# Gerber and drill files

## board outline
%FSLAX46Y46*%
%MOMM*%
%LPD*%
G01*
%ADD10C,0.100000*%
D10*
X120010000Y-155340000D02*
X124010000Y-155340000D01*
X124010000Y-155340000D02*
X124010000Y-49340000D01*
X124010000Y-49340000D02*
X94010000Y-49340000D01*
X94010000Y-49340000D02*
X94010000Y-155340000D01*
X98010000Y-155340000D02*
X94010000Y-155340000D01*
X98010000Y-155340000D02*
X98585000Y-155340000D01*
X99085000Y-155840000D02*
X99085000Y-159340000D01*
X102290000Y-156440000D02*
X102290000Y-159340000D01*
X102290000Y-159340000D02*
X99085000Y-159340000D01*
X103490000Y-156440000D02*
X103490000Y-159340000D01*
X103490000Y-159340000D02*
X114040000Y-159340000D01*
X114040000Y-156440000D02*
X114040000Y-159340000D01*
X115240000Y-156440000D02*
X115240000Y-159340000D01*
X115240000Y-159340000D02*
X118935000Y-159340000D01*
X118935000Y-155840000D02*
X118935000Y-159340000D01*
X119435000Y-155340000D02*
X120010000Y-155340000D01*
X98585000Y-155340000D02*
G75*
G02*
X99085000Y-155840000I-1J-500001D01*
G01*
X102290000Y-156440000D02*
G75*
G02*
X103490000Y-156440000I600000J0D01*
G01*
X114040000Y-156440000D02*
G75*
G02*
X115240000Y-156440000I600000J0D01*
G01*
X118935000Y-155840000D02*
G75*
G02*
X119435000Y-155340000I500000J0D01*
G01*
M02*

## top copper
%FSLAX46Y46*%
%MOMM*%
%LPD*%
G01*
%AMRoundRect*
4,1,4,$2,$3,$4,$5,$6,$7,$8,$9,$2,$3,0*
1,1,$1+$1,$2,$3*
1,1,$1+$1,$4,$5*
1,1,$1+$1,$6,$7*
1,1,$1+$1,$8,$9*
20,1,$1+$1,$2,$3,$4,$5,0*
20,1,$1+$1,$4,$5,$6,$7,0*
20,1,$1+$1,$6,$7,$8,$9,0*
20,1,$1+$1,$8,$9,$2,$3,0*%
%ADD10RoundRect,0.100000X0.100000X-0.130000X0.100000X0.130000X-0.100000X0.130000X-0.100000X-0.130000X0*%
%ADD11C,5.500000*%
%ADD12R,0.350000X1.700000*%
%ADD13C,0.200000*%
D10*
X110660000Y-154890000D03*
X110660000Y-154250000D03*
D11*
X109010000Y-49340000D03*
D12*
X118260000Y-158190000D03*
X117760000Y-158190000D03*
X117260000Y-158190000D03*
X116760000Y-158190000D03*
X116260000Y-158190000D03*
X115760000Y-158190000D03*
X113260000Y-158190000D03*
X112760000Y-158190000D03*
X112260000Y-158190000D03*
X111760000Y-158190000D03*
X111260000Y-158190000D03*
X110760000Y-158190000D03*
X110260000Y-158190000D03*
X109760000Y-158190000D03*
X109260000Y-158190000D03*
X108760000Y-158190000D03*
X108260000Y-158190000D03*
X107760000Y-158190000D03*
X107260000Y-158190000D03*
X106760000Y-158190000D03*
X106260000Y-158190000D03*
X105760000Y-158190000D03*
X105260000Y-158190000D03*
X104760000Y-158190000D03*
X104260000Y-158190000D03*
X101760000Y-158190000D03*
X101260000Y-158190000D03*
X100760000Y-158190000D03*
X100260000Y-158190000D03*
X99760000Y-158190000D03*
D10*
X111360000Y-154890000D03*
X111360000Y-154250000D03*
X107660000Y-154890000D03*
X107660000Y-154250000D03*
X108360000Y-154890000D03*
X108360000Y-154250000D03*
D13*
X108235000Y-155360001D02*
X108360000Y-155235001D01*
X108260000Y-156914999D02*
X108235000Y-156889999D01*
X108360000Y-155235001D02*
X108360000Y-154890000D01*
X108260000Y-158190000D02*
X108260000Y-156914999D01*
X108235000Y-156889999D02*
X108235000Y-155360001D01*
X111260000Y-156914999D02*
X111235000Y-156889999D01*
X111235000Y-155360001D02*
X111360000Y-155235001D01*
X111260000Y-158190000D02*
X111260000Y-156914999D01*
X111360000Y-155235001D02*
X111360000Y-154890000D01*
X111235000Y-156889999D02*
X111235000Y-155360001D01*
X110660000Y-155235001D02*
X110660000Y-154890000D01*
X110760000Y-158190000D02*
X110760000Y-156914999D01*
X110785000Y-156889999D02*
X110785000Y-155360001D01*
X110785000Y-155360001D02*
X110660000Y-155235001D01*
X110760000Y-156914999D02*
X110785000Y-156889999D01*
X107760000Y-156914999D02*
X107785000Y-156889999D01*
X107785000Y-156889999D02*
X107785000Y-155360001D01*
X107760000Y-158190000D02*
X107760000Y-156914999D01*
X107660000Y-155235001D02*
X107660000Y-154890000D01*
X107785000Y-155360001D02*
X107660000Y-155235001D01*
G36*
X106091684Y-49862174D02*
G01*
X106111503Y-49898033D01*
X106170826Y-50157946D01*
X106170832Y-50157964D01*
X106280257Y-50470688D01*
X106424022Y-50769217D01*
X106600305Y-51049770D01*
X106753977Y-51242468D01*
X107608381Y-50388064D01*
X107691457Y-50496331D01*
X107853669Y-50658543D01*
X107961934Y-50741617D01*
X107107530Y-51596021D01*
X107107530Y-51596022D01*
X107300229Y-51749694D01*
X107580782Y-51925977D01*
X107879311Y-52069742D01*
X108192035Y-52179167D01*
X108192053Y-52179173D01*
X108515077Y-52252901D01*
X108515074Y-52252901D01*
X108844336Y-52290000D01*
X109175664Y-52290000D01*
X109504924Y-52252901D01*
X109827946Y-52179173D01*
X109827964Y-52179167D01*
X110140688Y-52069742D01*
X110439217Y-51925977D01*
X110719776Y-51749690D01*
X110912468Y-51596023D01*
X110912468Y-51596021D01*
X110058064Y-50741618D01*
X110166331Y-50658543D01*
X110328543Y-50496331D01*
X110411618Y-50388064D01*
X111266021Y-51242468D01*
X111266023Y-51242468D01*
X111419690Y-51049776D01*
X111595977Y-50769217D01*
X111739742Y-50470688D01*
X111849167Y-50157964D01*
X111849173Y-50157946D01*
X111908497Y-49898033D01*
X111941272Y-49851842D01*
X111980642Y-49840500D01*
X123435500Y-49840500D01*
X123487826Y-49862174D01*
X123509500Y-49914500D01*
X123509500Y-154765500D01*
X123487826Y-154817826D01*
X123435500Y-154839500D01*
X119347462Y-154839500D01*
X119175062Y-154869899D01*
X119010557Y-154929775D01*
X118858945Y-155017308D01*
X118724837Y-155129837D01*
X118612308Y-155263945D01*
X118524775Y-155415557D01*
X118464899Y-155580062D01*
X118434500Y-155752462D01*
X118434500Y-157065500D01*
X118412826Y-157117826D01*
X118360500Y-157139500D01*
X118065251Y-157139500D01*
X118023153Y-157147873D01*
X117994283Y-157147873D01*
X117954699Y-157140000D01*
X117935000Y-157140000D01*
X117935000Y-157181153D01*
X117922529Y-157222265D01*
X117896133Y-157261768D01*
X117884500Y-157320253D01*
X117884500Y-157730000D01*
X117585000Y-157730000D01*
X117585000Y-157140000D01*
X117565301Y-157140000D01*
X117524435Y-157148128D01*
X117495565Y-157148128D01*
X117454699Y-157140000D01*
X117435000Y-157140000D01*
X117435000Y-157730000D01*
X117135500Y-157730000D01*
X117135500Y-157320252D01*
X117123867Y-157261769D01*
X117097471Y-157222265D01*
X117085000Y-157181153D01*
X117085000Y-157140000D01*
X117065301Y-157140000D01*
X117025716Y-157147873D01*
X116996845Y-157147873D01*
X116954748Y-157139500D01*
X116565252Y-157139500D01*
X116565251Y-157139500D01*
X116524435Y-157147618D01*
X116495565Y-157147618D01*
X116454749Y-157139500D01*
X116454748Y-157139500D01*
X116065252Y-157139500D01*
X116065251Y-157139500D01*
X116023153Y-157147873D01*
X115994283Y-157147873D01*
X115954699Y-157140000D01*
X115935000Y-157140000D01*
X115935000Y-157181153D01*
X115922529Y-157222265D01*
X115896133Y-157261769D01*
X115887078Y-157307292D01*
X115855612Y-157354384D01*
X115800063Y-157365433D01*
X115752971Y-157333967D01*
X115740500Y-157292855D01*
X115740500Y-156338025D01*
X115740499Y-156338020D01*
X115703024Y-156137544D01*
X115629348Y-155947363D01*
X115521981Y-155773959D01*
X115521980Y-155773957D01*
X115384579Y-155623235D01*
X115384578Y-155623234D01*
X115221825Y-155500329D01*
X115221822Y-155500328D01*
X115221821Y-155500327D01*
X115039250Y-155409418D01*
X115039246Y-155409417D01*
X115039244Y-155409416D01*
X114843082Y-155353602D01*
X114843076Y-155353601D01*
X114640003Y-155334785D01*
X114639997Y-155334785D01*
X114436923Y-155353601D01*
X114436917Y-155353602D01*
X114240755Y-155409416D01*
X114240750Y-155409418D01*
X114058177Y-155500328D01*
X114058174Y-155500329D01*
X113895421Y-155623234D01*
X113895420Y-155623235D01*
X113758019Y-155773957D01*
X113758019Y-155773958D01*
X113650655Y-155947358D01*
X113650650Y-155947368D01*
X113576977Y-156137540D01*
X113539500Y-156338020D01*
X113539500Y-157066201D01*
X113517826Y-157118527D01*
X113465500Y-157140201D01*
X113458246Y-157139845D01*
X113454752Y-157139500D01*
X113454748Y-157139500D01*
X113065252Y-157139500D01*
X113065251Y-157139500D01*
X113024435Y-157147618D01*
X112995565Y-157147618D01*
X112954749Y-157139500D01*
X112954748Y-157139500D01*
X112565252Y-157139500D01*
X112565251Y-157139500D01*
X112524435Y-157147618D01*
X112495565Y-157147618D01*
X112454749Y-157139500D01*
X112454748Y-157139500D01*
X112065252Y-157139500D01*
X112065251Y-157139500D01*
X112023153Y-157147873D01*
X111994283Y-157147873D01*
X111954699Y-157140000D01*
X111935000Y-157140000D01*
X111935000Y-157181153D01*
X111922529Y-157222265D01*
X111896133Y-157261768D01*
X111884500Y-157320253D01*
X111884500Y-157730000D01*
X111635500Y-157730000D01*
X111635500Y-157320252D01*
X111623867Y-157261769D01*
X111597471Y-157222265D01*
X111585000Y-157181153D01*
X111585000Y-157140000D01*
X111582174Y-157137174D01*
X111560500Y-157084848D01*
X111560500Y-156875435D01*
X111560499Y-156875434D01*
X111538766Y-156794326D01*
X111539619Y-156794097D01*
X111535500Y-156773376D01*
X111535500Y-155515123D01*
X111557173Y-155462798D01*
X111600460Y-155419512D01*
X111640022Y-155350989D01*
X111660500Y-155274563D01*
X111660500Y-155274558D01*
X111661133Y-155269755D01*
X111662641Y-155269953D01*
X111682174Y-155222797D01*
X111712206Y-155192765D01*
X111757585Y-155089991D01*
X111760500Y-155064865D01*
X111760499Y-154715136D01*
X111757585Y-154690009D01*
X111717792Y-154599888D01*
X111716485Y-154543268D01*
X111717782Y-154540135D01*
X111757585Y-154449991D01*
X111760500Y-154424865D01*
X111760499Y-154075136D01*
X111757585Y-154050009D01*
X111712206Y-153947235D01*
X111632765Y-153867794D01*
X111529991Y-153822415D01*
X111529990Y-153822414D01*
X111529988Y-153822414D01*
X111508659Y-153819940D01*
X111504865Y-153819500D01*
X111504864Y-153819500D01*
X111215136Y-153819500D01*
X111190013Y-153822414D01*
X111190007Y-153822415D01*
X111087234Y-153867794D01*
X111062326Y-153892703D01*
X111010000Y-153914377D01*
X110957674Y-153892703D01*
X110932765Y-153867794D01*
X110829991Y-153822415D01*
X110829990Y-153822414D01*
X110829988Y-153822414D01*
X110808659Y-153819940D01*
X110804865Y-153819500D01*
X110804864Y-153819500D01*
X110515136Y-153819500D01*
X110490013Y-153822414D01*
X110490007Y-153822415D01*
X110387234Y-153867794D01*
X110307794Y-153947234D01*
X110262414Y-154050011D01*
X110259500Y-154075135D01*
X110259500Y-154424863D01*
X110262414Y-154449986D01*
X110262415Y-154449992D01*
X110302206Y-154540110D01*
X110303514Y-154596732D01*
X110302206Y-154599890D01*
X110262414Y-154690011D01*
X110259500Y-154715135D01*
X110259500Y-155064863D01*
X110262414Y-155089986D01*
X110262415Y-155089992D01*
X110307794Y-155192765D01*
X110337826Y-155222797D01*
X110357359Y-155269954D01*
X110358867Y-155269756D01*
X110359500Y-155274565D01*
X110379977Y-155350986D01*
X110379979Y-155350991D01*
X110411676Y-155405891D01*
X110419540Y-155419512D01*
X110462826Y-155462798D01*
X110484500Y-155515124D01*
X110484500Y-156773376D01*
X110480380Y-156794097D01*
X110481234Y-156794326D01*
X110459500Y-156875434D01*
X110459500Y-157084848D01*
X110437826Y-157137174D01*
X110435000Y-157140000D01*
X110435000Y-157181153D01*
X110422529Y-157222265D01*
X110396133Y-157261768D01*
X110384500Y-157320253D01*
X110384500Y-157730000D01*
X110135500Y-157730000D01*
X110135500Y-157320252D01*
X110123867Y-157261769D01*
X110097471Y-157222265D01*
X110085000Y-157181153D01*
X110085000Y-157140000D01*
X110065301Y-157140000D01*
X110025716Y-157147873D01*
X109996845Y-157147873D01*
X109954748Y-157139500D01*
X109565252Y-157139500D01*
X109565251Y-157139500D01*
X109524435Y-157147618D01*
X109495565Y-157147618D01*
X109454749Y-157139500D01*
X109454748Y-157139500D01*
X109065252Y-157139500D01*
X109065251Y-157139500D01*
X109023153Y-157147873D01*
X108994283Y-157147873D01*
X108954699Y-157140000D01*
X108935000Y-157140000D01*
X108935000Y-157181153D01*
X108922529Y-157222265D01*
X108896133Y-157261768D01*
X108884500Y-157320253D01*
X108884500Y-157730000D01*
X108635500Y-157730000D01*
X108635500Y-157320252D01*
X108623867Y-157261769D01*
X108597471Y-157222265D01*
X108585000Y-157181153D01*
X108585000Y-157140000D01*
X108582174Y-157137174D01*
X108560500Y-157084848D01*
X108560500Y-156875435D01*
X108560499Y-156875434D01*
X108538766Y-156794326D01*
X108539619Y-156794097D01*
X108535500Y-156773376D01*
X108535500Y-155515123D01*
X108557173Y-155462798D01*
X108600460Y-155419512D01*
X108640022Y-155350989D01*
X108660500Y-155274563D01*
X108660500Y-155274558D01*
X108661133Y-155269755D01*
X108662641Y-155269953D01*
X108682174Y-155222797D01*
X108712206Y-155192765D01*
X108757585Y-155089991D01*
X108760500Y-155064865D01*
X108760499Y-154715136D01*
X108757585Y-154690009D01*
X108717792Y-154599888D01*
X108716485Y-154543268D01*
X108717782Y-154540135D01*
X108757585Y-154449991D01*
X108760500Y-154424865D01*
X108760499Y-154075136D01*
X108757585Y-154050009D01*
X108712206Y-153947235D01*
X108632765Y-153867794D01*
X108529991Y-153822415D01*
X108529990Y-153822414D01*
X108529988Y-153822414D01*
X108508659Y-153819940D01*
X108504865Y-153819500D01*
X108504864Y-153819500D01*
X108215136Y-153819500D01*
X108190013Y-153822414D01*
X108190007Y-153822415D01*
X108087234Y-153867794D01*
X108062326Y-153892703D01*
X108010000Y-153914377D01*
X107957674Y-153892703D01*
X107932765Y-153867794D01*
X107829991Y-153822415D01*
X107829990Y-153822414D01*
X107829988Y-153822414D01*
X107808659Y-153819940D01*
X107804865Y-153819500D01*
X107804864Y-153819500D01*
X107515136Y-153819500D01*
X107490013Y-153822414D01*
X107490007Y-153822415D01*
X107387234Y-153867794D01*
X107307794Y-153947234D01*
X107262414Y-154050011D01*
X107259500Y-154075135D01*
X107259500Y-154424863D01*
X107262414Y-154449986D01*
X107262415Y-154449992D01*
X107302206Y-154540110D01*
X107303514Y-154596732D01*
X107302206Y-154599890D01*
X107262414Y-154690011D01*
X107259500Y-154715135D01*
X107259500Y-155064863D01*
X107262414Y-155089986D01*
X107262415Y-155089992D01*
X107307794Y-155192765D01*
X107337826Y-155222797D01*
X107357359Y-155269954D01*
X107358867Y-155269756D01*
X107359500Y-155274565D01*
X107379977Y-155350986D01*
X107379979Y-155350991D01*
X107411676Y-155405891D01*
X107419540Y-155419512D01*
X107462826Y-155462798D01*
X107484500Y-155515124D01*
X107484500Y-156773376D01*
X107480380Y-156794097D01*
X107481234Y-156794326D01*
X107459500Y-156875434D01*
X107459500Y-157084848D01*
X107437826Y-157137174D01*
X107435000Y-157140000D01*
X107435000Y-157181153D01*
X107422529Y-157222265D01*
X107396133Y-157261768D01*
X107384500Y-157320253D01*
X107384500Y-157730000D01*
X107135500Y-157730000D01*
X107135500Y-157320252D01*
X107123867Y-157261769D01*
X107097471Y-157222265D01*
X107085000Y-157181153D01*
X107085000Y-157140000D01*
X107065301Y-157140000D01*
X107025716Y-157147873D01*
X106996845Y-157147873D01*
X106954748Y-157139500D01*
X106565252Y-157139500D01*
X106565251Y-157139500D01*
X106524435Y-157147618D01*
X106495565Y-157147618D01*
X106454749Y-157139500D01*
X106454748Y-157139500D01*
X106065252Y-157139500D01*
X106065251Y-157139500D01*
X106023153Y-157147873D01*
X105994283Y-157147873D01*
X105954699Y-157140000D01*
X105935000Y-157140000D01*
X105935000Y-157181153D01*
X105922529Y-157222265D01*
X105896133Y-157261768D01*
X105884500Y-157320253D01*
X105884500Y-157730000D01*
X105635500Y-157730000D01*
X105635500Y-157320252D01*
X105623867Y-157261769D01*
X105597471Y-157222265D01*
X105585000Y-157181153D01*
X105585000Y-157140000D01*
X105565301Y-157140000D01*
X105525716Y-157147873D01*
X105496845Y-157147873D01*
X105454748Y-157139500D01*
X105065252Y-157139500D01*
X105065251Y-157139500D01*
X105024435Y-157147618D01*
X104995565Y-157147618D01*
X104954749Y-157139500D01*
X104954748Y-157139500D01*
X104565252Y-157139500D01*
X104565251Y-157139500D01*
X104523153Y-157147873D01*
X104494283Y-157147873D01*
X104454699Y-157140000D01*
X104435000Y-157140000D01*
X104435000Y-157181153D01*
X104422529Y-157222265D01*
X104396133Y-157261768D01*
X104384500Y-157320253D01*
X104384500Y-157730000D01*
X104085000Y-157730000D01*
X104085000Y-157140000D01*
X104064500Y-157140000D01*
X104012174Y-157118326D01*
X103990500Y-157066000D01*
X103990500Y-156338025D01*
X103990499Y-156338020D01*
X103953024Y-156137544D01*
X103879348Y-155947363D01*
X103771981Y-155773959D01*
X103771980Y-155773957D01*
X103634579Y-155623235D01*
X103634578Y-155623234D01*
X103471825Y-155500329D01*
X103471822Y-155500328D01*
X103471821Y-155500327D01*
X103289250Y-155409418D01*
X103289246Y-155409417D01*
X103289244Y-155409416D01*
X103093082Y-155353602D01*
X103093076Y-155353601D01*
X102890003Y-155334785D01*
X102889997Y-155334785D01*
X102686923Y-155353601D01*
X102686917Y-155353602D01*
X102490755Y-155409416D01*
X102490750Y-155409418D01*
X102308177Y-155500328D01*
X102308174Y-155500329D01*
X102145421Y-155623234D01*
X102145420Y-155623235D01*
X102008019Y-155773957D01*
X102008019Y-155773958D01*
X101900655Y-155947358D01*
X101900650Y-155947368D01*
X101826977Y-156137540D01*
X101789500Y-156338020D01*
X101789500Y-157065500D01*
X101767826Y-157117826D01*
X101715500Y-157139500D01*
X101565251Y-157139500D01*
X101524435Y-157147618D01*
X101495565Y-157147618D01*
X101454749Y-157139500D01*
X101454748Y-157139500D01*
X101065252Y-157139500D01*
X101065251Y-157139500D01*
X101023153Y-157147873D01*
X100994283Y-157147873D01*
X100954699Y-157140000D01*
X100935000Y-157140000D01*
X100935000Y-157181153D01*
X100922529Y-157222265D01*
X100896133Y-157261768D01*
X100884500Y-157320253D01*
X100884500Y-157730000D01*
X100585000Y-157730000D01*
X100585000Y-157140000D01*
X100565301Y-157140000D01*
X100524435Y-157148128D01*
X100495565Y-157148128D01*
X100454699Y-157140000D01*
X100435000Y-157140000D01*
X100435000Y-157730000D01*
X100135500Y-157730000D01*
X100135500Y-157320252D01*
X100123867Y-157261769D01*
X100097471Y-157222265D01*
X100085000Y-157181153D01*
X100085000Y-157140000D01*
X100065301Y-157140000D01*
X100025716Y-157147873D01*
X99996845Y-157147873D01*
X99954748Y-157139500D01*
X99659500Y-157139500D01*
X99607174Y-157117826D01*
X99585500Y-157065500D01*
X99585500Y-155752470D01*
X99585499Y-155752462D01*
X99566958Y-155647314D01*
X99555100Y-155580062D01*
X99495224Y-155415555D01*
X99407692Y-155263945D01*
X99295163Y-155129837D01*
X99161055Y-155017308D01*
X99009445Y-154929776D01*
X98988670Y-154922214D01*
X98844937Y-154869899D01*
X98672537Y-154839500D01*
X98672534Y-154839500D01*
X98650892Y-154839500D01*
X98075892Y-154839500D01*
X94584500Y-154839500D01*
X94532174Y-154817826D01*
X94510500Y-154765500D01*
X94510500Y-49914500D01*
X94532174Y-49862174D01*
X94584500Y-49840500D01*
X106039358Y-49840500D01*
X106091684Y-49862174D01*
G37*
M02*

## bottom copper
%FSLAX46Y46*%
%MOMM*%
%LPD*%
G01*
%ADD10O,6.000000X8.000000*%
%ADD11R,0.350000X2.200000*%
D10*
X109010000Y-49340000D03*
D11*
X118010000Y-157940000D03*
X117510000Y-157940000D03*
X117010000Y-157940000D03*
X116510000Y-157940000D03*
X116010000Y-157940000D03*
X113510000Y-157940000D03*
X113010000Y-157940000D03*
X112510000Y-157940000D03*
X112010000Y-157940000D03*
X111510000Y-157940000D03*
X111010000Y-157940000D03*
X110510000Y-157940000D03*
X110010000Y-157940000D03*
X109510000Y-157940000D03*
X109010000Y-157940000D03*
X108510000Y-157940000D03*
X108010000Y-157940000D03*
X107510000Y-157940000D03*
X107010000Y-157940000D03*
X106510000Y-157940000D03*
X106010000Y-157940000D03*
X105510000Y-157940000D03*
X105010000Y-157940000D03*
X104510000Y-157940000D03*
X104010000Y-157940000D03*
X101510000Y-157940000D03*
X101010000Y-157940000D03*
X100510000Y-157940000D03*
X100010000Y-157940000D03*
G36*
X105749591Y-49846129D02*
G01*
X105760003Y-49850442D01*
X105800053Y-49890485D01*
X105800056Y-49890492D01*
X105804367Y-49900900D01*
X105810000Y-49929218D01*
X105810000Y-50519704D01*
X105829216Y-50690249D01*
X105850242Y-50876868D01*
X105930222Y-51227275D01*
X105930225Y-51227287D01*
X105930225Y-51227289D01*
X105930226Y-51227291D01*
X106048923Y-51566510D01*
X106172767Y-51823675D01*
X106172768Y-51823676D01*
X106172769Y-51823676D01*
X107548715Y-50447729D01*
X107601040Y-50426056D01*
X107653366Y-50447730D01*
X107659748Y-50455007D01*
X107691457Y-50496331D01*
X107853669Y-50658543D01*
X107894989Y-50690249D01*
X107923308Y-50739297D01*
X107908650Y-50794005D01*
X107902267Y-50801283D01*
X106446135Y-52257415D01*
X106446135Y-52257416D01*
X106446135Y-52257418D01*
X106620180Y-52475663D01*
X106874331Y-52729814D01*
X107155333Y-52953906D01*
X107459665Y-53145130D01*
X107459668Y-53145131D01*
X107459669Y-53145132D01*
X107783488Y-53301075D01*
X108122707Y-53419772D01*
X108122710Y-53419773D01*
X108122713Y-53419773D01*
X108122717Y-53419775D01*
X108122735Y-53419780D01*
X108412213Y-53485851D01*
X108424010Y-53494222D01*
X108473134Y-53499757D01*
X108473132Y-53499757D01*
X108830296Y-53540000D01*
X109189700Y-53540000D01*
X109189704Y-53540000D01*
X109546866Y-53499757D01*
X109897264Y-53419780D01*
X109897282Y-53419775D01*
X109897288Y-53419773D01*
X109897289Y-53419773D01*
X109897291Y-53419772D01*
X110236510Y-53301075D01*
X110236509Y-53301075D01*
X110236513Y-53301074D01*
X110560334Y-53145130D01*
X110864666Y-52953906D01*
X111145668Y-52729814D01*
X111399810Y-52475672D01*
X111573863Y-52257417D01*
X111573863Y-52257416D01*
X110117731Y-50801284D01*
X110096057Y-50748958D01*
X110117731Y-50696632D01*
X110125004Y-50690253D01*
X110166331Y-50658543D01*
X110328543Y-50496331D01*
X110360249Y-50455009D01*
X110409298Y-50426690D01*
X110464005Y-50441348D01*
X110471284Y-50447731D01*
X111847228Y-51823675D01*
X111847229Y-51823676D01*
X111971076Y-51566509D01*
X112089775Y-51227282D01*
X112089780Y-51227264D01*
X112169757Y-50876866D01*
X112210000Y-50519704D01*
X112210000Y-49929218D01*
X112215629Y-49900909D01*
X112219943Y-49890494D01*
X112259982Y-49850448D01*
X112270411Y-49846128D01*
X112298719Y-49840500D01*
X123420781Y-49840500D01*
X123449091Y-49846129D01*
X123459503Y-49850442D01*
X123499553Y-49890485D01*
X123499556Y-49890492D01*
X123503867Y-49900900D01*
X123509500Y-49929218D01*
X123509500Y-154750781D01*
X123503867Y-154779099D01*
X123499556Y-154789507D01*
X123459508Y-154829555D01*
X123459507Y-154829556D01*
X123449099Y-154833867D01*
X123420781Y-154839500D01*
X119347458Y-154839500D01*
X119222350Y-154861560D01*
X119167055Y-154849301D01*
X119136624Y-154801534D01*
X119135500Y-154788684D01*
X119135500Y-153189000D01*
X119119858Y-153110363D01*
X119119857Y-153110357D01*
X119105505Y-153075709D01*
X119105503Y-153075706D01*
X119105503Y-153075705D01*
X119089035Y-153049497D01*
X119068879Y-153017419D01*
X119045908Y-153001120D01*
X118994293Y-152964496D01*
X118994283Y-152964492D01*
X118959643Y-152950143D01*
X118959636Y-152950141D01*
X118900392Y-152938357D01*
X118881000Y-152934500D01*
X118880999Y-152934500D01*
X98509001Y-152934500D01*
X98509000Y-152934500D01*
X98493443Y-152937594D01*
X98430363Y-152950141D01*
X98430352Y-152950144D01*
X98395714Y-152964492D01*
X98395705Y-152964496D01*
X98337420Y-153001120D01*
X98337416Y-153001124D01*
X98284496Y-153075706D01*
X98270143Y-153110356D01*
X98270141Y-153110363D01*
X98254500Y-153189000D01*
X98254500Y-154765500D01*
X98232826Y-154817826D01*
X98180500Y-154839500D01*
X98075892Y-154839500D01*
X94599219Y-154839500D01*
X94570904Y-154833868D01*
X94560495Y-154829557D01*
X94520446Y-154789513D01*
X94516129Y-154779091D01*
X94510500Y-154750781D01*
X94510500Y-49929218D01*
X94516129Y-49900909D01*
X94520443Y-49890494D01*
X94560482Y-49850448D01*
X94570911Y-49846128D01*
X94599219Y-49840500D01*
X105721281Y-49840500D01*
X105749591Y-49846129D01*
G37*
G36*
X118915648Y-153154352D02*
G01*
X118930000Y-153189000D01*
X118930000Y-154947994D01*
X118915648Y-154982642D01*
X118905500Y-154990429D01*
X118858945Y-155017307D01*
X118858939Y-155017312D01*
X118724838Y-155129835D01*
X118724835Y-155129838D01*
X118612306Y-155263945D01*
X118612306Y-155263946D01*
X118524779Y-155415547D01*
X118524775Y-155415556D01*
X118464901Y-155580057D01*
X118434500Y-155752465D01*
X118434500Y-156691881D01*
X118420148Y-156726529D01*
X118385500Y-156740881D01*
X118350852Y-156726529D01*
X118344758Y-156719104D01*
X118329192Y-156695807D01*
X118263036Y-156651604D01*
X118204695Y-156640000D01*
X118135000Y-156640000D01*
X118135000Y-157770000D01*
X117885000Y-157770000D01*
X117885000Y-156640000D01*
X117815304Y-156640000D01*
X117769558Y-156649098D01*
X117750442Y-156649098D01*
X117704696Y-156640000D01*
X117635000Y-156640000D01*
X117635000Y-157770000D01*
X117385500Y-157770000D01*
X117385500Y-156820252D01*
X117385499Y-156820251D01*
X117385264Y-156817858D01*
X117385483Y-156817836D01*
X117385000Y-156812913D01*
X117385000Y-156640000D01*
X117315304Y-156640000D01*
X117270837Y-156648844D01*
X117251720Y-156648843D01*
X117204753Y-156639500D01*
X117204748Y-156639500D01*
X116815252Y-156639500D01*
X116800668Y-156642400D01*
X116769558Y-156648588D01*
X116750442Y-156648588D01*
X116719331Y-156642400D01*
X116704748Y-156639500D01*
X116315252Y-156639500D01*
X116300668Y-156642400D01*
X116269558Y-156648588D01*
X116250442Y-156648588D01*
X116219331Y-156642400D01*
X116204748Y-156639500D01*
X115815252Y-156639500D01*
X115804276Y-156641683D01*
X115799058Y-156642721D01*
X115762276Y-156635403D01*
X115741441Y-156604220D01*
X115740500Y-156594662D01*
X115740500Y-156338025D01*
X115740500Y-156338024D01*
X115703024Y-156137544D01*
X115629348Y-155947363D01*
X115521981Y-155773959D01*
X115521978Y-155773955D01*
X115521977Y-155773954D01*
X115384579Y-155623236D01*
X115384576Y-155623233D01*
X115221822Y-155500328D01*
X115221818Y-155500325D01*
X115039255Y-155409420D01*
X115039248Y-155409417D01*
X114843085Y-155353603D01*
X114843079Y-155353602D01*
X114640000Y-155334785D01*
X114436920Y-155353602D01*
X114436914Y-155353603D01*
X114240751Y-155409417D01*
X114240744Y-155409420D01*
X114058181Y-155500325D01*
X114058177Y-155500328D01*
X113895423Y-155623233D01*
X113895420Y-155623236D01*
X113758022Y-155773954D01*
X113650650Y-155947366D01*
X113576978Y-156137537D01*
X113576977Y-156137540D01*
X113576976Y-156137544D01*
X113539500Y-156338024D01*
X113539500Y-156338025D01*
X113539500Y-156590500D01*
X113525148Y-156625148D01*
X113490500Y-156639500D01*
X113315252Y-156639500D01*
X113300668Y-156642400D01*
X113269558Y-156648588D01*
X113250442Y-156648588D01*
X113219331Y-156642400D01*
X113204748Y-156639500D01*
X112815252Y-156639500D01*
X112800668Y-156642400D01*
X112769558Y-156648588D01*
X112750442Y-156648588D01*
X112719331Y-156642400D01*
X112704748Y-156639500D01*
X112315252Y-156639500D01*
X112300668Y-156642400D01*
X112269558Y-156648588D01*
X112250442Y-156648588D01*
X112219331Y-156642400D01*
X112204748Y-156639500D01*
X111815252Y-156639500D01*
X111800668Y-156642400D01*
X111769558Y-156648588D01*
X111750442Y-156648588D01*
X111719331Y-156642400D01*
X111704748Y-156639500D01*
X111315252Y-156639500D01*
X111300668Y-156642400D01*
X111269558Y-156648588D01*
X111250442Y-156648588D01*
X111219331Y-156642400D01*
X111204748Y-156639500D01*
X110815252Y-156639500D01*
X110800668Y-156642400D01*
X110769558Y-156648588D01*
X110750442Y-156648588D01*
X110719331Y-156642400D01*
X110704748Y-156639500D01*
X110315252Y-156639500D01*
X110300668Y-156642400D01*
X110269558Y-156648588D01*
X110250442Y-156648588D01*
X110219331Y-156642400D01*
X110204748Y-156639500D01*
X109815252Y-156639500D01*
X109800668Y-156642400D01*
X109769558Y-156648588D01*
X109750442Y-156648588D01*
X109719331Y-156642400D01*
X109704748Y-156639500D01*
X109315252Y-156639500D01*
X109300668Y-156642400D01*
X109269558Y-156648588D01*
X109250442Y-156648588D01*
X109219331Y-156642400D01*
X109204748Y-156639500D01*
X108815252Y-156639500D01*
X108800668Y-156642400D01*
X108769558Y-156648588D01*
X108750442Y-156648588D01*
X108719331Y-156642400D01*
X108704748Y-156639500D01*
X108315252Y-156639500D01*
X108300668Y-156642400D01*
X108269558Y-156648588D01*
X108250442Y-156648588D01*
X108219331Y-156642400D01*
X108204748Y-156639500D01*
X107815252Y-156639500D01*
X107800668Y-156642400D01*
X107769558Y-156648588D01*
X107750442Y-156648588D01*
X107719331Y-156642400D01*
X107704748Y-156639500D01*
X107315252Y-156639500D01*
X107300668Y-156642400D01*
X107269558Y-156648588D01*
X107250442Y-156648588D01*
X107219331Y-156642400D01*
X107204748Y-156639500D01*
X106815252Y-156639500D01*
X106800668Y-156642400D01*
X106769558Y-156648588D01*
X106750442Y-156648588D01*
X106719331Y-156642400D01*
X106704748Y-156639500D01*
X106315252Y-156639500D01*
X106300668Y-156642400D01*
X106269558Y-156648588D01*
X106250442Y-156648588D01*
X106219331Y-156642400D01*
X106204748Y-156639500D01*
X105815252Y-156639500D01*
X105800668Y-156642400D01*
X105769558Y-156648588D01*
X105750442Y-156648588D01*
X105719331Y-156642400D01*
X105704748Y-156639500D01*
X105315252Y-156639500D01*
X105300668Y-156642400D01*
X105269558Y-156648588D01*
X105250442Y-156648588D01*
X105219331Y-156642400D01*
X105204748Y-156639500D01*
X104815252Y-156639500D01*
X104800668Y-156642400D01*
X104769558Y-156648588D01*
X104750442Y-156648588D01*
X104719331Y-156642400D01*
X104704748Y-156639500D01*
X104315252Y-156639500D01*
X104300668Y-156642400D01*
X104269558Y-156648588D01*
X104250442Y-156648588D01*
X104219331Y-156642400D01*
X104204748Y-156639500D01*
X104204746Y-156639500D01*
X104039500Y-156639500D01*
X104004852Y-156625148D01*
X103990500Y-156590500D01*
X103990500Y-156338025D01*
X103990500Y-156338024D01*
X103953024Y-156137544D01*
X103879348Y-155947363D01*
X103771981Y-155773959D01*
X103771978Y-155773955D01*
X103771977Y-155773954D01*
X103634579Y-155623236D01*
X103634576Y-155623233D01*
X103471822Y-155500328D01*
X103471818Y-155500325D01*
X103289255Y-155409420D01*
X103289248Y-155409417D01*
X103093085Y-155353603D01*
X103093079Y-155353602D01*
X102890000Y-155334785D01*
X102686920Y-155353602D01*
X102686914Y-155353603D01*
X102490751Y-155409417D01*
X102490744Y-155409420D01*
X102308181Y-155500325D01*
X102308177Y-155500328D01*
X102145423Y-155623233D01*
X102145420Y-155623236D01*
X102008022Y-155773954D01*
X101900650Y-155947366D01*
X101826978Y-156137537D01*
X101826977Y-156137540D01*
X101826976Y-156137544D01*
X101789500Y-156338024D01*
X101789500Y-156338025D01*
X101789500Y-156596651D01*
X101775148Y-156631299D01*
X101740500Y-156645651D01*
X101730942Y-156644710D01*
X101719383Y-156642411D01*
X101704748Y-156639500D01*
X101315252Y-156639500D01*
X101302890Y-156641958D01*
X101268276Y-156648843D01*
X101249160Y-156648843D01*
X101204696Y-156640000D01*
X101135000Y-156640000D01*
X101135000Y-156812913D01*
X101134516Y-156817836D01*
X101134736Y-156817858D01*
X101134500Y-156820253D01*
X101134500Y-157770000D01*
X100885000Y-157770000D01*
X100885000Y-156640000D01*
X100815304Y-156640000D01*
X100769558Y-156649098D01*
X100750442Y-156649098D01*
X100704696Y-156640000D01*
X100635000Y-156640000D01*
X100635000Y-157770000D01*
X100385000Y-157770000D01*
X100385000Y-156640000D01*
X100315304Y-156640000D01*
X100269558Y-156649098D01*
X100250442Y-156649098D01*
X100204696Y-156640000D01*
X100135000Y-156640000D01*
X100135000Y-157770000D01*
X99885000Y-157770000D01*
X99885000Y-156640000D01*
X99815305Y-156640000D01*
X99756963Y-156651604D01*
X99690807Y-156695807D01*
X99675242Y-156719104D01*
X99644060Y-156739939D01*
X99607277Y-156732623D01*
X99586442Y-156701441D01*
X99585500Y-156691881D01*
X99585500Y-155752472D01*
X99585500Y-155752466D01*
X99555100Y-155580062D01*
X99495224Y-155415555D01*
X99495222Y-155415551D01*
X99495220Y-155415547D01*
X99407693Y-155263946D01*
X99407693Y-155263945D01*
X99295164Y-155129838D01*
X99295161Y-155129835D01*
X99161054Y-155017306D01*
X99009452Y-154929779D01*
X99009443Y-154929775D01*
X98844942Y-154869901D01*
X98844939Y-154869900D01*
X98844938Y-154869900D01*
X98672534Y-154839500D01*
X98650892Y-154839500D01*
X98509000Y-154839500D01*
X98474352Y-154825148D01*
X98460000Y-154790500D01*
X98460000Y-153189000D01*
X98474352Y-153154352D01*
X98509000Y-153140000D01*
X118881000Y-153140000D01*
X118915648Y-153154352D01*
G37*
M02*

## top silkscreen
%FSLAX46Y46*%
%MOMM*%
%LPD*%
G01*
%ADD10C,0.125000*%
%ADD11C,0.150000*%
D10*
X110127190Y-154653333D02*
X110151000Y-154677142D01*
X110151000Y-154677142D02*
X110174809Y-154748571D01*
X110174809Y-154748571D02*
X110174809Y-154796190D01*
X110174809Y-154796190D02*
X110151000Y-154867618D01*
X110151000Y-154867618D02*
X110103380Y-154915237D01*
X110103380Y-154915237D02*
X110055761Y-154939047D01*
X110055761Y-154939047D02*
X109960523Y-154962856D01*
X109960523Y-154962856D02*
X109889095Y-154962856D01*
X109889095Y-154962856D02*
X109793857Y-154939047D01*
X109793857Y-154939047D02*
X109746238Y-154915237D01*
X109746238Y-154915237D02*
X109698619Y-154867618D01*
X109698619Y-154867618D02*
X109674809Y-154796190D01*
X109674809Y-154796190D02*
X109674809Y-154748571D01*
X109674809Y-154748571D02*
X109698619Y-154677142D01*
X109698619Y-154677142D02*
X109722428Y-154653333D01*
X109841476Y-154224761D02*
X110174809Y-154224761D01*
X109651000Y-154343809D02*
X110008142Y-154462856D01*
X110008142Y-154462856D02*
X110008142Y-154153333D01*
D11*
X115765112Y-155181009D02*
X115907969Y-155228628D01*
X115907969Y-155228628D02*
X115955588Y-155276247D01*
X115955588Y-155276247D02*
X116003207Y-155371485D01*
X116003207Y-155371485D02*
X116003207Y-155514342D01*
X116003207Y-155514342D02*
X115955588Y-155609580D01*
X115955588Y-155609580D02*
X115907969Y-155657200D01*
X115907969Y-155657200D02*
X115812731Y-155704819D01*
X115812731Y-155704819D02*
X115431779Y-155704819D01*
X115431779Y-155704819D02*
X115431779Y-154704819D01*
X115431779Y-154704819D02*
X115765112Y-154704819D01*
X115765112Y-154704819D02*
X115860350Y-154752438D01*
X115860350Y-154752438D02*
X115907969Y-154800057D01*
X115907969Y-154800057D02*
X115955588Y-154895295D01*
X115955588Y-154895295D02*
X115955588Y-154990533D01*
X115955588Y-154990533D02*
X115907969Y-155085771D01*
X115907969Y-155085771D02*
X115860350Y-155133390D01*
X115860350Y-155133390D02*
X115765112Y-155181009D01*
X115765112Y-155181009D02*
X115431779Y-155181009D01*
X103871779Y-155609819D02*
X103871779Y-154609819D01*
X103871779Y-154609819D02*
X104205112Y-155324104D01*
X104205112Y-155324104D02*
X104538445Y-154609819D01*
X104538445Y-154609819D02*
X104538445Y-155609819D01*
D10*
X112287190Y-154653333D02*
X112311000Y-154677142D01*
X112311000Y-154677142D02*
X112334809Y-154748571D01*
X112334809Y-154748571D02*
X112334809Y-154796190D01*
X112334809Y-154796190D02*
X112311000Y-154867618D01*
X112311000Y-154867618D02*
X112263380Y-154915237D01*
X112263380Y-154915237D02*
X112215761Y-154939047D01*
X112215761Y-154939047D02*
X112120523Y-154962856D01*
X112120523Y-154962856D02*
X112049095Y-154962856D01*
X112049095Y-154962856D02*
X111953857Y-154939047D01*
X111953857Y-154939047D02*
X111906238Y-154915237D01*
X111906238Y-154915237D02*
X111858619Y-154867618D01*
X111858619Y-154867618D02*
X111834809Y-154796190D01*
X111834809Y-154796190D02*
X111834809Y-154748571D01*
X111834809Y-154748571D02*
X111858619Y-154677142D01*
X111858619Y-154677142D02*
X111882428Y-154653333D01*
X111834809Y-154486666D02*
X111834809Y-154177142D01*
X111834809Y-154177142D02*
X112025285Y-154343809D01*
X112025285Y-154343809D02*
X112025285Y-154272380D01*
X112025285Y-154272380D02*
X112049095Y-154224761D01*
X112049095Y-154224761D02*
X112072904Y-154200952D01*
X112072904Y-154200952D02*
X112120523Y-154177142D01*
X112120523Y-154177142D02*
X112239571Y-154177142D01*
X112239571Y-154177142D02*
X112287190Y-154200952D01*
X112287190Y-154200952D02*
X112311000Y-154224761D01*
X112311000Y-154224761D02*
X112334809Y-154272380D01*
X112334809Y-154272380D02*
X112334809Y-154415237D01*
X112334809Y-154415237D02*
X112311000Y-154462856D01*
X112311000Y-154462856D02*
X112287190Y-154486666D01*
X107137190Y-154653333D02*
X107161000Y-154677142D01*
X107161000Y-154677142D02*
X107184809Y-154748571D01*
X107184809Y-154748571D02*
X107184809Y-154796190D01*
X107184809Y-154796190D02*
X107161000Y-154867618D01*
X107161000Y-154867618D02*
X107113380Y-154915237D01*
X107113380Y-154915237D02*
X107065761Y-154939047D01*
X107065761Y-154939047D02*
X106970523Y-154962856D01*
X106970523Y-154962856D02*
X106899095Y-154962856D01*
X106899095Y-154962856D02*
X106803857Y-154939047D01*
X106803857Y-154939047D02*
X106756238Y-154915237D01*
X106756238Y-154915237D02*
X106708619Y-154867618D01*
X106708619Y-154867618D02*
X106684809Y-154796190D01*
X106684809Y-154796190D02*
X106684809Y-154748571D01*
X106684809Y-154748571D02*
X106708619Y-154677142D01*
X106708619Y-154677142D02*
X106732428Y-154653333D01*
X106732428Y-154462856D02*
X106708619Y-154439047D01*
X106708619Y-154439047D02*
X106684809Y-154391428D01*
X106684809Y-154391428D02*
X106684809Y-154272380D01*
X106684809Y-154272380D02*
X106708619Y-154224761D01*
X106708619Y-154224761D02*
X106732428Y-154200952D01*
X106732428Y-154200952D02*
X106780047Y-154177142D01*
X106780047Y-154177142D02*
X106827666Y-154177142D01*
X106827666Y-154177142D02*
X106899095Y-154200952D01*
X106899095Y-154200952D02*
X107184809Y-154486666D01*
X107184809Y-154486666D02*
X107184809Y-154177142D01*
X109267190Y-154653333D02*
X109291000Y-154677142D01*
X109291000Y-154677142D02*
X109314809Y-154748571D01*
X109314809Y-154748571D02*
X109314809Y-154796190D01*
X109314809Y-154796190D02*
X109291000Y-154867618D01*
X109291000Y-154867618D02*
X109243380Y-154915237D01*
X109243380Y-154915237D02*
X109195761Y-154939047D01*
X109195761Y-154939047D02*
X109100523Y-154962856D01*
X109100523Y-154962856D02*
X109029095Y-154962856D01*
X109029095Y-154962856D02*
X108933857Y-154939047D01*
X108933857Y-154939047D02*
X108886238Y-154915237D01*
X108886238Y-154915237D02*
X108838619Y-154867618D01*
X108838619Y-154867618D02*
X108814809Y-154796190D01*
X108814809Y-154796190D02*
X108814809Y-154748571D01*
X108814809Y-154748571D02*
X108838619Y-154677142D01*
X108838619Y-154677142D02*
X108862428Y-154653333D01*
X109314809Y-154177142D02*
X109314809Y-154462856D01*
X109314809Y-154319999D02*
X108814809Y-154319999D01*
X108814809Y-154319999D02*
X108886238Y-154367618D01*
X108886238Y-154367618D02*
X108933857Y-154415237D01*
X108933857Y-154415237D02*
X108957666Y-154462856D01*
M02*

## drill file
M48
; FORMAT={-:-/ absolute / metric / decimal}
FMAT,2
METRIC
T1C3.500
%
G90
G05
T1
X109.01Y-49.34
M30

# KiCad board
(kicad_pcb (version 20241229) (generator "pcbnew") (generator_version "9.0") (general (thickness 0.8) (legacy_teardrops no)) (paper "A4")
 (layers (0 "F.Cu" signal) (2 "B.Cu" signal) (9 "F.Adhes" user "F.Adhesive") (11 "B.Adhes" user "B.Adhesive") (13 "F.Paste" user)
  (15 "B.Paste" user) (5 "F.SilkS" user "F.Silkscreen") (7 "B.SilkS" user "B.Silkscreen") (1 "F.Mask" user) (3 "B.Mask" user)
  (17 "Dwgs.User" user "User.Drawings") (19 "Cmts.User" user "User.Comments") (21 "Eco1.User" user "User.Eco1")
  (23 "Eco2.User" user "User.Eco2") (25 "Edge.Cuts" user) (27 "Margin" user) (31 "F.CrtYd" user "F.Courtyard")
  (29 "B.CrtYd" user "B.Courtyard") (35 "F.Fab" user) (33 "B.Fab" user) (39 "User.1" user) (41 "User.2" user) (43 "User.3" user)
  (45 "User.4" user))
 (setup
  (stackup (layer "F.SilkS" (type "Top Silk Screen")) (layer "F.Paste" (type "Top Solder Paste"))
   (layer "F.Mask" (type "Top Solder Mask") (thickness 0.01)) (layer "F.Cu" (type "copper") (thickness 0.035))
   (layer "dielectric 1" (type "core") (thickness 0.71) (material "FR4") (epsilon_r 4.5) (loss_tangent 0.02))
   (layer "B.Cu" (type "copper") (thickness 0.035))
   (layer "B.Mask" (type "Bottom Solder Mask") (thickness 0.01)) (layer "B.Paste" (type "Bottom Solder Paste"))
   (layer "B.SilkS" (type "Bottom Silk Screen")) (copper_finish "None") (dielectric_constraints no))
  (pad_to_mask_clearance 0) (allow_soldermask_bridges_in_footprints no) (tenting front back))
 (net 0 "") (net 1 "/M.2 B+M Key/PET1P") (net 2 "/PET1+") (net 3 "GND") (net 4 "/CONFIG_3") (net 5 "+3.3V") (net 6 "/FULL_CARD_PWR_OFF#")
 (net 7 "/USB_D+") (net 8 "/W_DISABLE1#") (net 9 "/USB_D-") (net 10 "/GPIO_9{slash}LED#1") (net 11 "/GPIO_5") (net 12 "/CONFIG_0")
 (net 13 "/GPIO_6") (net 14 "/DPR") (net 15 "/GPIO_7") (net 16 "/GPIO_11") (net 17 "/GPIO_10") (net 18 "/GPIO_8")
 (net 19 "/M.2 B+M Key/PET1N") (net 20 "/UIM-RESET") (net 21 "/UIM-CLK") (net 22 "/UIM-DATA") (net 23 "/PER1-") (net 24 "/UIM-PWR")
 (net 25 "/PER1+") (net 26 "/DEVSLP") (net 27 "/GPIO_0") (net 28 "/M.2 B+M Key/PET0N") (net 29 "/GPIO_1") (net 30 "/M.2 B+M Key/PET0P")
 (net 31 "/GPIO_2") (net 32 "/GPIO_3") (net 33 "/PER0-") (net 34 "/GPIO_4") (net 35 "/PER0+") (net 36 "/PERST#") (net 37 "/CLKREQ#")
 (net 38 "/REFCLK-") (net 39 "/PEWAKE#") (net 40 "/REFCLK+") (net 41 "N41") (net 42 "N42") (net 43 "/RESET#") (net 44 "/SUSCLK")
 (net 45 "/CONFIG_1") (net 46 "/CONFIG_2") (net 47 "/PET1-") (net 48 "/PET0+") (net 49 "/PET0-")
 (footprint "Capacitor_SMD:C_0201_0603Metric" (layer "F.Cu") (at 110.66 154.57 90)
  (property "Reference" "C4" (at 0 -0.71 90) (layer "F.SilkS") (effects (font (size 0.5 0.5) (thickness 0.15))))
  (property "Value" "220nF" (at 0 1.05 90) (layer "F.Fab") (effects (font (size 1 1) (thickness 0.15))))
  (pad "" smd roundrect (at -0.345 0 90) (size 0.318 0.36) (layers "F.Paste") (roundrect_rratio 0.25))
  (pad "" smd roundrect (at 0.345 0 90) (size 0.318 0.36) (layers "F.Paste") (roundrect_rratio 0.25))
  (pad "1" smd roundrect (at -0.32 0 90) (size 0.46 0.4) (layers "F.Cu" "F.Mask") (roundrect_rratio 0.25) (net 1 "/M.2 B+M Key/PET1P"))
  (pad "2" smd roundrect (at 0.32 0 90) (size 0.46 0.4) (layers "F.Cu" "F.Mask") (roundrect_rratio 0.25) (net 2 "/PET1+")))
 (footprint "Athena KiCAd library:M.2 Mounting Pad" (layer "F.Cu") (at 109.01 49.34)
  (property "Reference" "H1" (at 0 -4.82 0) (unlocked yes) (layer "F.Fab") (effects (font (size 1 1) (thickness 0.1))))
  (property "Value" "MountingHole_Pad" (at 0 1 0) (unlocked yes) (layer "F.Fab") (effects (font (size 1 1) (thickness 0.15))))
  (pad "1" thru_hole circle (at 0 0) (size 5.5 5.5) (drill 3.5) (layers "*.Cu" "*.Mask") (remove_unused_layers no) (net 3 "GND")
   (padstack (mode front_inner_back)
    (layer "Inner" (shape circle) (size 5.5 5.5) (zone_connect -1))
    (layer "B.Cu" (shape oval) (size 6 8) (thermal_bridge_angle 45) (zone_connect -1)))))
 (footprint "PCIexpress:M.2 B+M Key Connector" (layer "F.Cu") (at 109.01 158.23)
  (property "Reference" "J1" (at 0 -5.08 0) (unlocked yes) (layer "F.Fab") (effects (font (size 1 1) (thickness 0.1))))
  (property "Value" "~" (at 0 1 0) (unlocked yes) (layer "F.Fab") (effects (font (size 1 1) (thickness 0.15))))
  (fp_line (start -11 -2.89) (end -10.425 -2.89) (stroke (width 0.1) (type default)) (layer "Edge.Cuts"))
  (fp_line (start -9.925 -2.39) (end -9.925 1.11) (stroke (width 0.1) (type default)) (layer "Edge.Cuts"))
  (fp_line (start -6.72 -1.79) (end -6.72 1.11) (stroke (width 0.1) (type default)) (layer "Edge.Cuts"))
  (fp_line (start -6.72 1.11) (end -9.925 1.11) (stroke (width 0.1) (type default)) (layer "Edge.Cuts"))
  (fp_line (start -5.52 -1.79) (end -5.52 1.11) (stroke (width 0.1) (type default)) (layer "Edge.Cuts"))
  (fp_line (start -5.52 1.11) (end 5.03 1.11) (stroke (width 0.1) (type default)) (layer "Edge.Cuts"))
  (fp_line (start 5.03 -1.79) (end 5.03 1.11) (stroke (width 0.1) (type default)) (layer "Edge.Cuts"))
  (fp_line (start 6.23 -1.79) (end 6.23 1.11) (stroke (width 0.1) (type default)) (layer "Edge.Cuts"))
  (fp_line (start 6.23 1.11) (end 9.925 1.11) (stroke (width 0.1) (type default)) (layer "Edge.Cuts"))
  (fp_line (start 9.925 -2.39) (end 9.925 1.11) (stroke (width 0.1) (type default)) (layer "Edge.Cuts"))
  (fp_line (start 10.425 -2.89) (end 11 -2.89) (stroke (width 0.1) (type default)) (layer "Edge.Cuts"))
  (fp_arc (start -10.425 -2.89) (mid -10.071447 -2.743553) (end -9.925 -2.39) (stroke (width 0.1) (type default)) (layer "Edge.Cuts"))
  (fp_arc (start -6.72 -1.79) (mid -6.12 -2.39) (end -5.52 -1.79) (stroke (width 0.1) (type default)) (layer "Edge.Cuts"))
  (fp_arc (start 5.03 -1.79) (mid 5.63 -2.39) (end 6.23 -1.79) (stroke (width 0.1) (type default)) (layer "Edge.Cuts"))
  (fp_arc (start 9.925 -2.39) (mid 10.071447 -2.743553) (end 10.425 -2.89) (stroke (width 0.1) (type default)) (layer "Edge.Cuts"))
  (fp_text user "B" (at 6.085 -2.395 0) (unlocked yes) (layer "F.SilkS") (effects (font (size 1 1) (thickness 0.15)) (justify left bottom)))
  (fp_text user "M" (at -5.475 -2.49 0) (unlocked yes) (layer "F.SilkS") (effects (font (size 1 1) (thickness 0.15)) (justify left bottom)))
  (pad "1" smd rect (at 9.25 -0.04 180) (size 0.35 1.7) (layers "F.Cu") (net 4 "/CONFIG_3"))
  (pad "2" smd rect (at 9 -0.29 180) (size 0.35 2.2) (layers "B.Cu") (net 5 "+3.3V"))
  (pad "3" smd rect (at 8.75 -0.04 180) (size 0.35 1.7) (layers "F.Cu") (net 3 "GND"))
  (pad "4" smd rect (at 8.5 -0.29 180) (size 0.35 2.2) (layers "B.Cu") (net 5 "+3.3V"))
  (pad "5" smd rect (at 8.25 -0.04 180) (size 0.35 1.7) (layers "F.Cu") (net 3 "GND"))
  (pad "6" smd rect (at 8 -0.29 180) (size 0.35 2.2) (layers "B.Cu") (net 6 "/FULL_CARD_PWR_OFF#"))
  (pad "7" smd rect (at 7.75 -0.04 180) (size 0.35 1.7) (layers "F.Cu") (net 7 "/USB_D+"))
  (pad "8" smd rect (at 7.5 -0.29 180) (size 0.35 2.2) (layers "B.Cu") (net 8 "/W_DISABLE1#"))
  (pad "9" smd rect (at 7.25 -0.04 180) (size 0.35 1.7) (layers "F.Cu") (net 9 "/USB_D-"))
  (pad "10" smd rect (at 7 -0.29 180) (size 0.35 2.2) (layers "B.Cu") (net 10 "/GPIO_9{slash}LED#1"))
  (pad "11" smd rect (at 6.75 -0.04 180) (size 0.35 1.7) (layers "F.Cu") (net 3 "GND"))
  (pad "20" smd rect (at 4.5 -0.29 180) (size 0.35 2.2) (layers "B.Cu") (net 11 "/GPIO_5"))
  (pad "21" smd rect (at 4.25 -0.04 180) (size 0.35 1.7) (layers "F.Cu") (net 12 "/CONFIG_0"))
  (pad "22" smd rect (at 4 -0.29 180) (size 0.35 2.2) (layers "B.Cu") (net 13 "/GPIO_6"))
  (pad "23" smd rect (at 3.75 -0.04 180) (size 0.35 1.7) (layers "F.Cu") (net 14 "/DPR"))
  (pad "24" smd rect (at 3.5 -0.29 180) (size 0.35 2.2) (layers "B.Cu") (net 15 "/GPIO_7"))
  (pad "25" smd rect (at 3.25 -0.04 180) (size 0.35 1.7) (layers "F.Cu") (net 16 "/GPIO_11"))
  (pad "26" smd rect (at 3 -0.29 180) (size 0.35 2.2) (layers "B.Cu") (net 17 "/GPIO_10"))
  (pad "27" smd rect (at 2.75 -0.04 180) (size 0.35 1.7) (layers "F.Cu") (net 3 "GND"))
  (pad "28" smd rect (at 2.5 -0.29 180) (size 0.35 2.2) (layers "B.Cu") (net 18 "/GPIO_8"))
  (pad "29" smd rect (at 2.25 -0.04 180) (size 0.35 1.7) (layers "F.Cu") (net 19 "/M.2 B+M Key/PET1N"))
  (pad "30" smd rect (at 2 -0.29 180) (size 0.35 2.2) (layers "B.Cu") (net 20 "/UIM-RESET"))
  (pad "31" smd rect (at 1.75 -0.04 180) (size 0.35 1.7) (layers "F.Cu") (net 1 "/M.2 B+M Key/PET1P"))
  (pad "32" smd rect (at 1.5 -0.29 180) (size 0.35 2.2) (layers "B.Cu") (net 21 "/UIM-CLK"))
  (pad "33" smd rect (at 1.25 -0.04 180) (size 0.35 1.7) (layers "F.Cu") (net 3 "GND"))
  (pad "34" smd rect (at 1 -0.29 180) (size 0.35 2.2) (layers "B.Cu") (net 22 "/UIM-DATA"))
  (pad "35" smd rect (at 0.75 -0.04 180) (size 0.35 1.7) (layers "F.Cu") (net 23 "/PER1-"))
  (pad "36" smd rect (at 0.5 -0.29 180) (size 0.35 2.2) (layers "B.Cu") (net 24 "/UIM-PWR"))
  (pad "37" smd rect (at 0.25 -0.04 180) (size 0.35 1.7) (layers "F.Cu") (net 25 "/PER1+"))
  (pad "38" smd rect (at 0 -0.29 180) (size 0.35 2.2) (layers "B.Cu") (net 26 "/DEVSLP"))
  (pad "39" smd rect (at -0.25 -0.04 180) (size 0.35 1.7) (layers "F.Cu") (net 3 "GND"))
  (pad "40" smd rect (at -0.5 -0.29 180) (size 0.35 2.2) (layers "B.Cu") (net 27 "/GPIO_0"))
  (pad "41" smd rect (at -0.75 -0.04 180) (size 0.35 1.7) (layers "F.Cu") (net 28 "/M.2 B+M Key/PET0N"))
  (pad "42" smd rect (at -1 -0.29 180) (size 0.35 2.2) (layers "B.Cu") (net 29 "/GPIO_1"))
  (pad "43" smd rect (at -1.25 -0.04 180) (size 0.35 1.7) (layers "F.Cu") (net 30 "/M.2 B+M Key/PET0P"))
  (pad "44" smd rect (at -1.5 -0.29 180) (size 0.35 2.2) (layers "B.Cu") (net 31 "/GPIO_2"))
  (pad "45" smd rect (at -1.75 -0.04 180) (size 0.35 1.7) (layers "F.Cu") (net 3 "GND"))
  (pad "46" smd rect (at -2 -0.29 180) (size 0.35 2.2) (layers "B.Cu") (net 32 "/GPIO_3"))
  (pad "47" smd rect (at -2.25 -0.04 180) (size 0.35 1.7) (layers "F.Cu") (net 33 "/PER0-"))
  (pad "48" smd rect (at -2.5 -0.29 180) (size 0.35 2.2) (layers "B.Cu") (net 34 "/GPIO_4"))
  (pad "49" smd rect (at -2.75 -0.04 180) (size 0.35 1.7) (layers "F.Cu") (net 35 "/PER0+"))
  (pad "50" smd rect (at -3 -0.29 180) (size 0.35 2.2) (layers "B.Cu") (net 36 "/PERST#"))
  (pad "51" smd rect (at -3.25 -0.04 180) (size 0.35 1.7) (layers "F.Cu") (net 3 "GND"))
  (pad "52" smd rect (at -3.5 -0.29 180) (size 0.35 2.2) (layers "B.Cu") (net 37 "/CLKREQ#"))
  (pad "53" smd rect (at -3.75 -0.04 180) (size 0.35 1.7) (layers "F.Cu") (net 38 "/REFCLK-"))
  (pad "54" smd rect (at -4 -0.29 180) (size 0.35 2.2) (layers "B.Cu") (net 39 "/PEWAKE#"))
  (pad "55" smd rect (at -4.25 -0.04 180) (size 0.35 1.7) (layers "F.Cu") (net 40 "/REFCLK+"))
  (pad "56" smd rect (at -4.5 -0.29 180) (size 0.35 2.2) (layers "B.Cu") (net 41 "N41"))
  (pad "57" smd rect (at -4.75 -0.04 180) (size 0.35 1.7) (layers "F.Cu") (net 3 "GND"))
  (pad "58" smd rect (at -5 -0.29 180) (size 0.35 2.2) (layers "B.Cu") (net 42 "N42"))
  (pad "67" smd rect (at -7.25 -0.04 180) (size 0.35 1.7) (layers "F.Cu") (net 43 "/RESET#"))
  (pad "68" smd rect (at -7.5 -0.29 180) (size 0.35 2.2) (layers "B.Cu") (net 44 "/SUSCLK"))
  (pad "69" smd rect (at -7.75 -0.04 180) (size 0.35 1.7) (layers "F.Cu") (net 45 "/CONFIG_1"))
  (pad "70" smd rect (at -8 -0.29 180) (size 0.35 2.2) (layers "B.Cu") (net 5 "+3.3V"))
  (pad "71" smd rect (at -8.25 -0.04 180) (size 0.35 1.7) (layers "F.Cu") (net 3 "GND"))
  (pad "72" smd rect (at -8.5 -0.29 180) (size 0.35 2.2) (layers "B.Cu") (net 5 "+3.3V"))
  (pad "73" smd rect (at -8.75 -0.04 180) (size 0.35 1.7) (layers "F.Cu") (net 3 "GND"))
  (pad "74" smd rect (at -9 -0.29 180) (size 0.35 2.2) (layers "B.Cu") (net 5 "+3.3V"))
  (pad "75" smd rect (at -9.25 -0.04 180) (size 0.35 1.7) (layers "F.Cu") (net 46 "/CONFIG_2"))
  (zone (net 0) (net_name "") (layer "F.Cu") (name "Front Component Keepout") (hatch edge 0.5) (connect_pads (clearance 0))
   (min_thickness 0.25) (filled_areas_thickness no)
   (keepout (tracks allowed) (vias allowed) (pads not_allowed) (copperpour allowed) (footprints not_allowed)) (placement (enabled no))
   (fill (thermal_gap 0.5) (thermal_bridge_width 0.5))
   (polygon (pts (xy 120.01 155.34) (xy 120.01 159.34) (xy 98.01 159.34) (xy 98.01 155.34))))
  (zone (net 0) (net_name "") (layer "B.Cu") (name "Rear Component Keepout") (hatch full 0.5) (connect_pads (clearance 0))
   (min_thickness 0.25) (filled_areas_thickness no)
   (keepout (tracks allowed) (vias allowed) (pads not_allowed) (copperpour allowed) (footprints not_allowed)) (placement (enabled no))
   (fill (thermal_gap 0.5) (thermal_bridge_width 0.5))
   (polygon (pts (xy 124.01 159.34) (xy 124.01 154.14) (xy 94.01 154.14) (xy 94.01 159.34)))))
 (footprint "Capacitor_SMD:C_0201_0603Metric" (layer "F.Cu") (at 111.36 154.57 90)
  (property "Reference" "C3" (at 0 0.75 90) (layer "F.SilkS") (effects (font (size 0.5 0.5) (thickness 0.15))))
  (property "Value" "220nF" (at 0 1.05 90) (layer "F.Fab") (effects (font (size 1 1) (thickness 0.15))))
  (pad "" smd roundrect (at -0.345 0 90) (size 0.318 0.36) (layers "F.Paste") (roundrect_rratio 0.25))
  (pad "" smd roundrect (at 0.345 0 90) (size 0.318 0.36) (layers "F.Paste") (roundrect_rratio 0.25))
  (pad "1" smd roundrect (at -0.32 0 90) (size 0.46 0.4) (layers "F.Cu" "F.Mask") (roundrect_rratio 0.25) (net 19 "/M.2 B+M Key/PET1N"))
  (pad "2" smd roundrect (at 0.32 0 90) (size 0.46 0.4) (layers "F.Cu" "F.Mask") (roundrect_rratio 0.25) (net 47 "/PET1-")))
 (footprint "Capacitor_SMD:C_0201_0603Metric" (layer "F.Cu") (at 107.66 154.57 90)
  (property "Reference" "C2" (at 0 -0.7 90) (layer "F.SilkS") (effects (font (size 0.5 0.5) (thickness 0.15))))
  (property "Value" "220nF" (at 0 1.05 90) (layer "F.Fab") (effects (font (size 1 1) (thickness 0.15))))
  (pad "" smd roundrect (at -0.345 0 90) (size 0.318 0.36) (layers "F.Paste") (roundrect_rratio 0.25))
  (pad "" smd roundrect (at 0.345 0 90) (size 0.318 0.36) (layers "F.Paste") (roundrect_rratio 0.25))
  (pad "1" smd roundrect (at -0.32 0 90) (size 0.46 0.4) (layers "F.Cu" "F.Mask") (roundrect_rratio 0.25) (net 30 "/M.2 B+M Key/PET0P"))
  (pad "2" smd roundrect (at 0.32 0 90) (size 0.46 0.4) (layers "F.Cu" "F.Mask") (roundrect_rratio 0.25) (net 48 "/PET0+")))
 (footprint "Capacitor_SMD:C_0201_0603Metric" (layer "F.Cu") (at 108.36 154.57 90)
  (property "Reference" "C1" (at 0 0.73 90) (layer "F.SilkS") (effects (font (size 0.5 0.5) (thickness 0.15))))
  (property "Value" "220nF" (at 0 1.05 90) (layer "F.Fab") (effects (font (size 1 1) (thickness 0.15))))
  (pad "" smd roundrect (at -0.345 0 90) (size 0.318 0.36) (layers "F.Paste") (roundrect_rratio 0.25))
  (pad "" smd roundrect (at 0.345 0 90) (size 0.318 0.36) (layers "F.Paste") (roundrect_rratio 0.25))
  (pad "1" smd roundrect (at -0.32 0 90) (size 0.46 0.4) (layers "F.Cu" "F.Mask") (roundrect_rratio 0.25) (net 28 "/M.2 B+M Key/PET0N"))
  (pad "2" smd roundrect (at 0.32 0 90) (size 0.46 0.4) (layers "F.Cu" "F.Mask") (roundrect_rratio 0.25) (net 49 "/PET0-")))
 (gr_line (start 120.01 155.34) (end 124.01 155.34) (stroke (width 0.1) (type default)) (layer "Edge.Cuts"))
 (gr_line (start 124.01 155.34) (end 124.01 49.34) (stroke (width 0.1) (type default)) (layer "Edge.Cuts"))
 (gr_line (start 124.01 49.34) (end 94.01 49.34) (stroke (width 0.1) (type default)) (layer "Edge.Cuts"))
 (gr_line (start 94.01 49.34) (end 94.01 155.34) (stroke (width 0.1) (type default)) (layer "Edge.Cuts"))
 (gr_line (start 98.01 155.34) (end 94.01 155.34) (stroke (width 0.1) (type default)) (layer "Edge.Cuts"))
 (segment (start 108.235 155.360001) (end 108.36 155.235001) (width 0.2) (layer "F.Cu") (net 28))
 (segment (start 108.26 156.914999) (end 108.235 156.889999) (width 0.2) (layer "F.Cu") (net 28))
 (segment (start 108.36 155.235001) (end 108.36 154.89) (width 0.2) (layer "F.Cu") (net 28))
 (segment (start 108.26 158.19) (end 108.26 156.914999) (width 0.2) (layer "F.Cu") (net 28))
 (segment (start 108.235 156.889999) (end 108.235 155.360001) (width 0.2) (layer "F.Cu") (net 28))
 (segment (start 111.26 156.914999) (end 111.235 156.889999) (width 0.2) (layer "F.Cu") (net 19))
 (segment (start 111.235 155.360001) (end 111.36 155.235001) (width 0.2) (layer "F.Cu") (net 19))
 (segment (start 111.26 158.19) (end 111.26 156.914999) (width 0.2) (layer "F.Cu") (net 19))
 (segment (start 111.36 155.235001) (end 111.36 154.89) (width 0.2) (layer "F.Cu") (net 19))
 (segment (start 111.235 156.889999) (end 111.235 155.360001) (width 0.2) (layer "F.Cu") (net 19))
 (segment (start 110.66 155.235001) (end 110.66 154.89) (width 0.2) (layer "F.Cu") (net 1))
 (segment (start 110.76 158.19) (end 110.76 156.914999) (width 0.2) (layer "F.Cu") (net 1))
 (segment (start 110.785 156.889999) (end 110.785 155.360001) (width 0.2) (layer "F.Cu") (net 1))
 (segment (start 110.785 155.360001) (end 110.66 155.235001) (width 0.2) (layer "F.Cu") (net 1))
 (segment (start 110.76 156.914999) (end 110.785 156.889999) (width 0.2) (layer "F.Cu") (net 1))
 (segment (start 107.76 156.914999) (end 107.785 156.889999) (width 0.2) (layer "F.Cu") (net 30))
 (segment (start 107.785 156.889999) (end 107.785 155.360001) (width 0.2) (layer "F.Cu") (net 30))
 (segment (start 107.76 158.19) (end 107.76 156.914999) (width 0.2) (layer "F.Cu") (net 30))
 (segment (start 107.66 155.235001) (end 107.66 154.89) (width 0.2) (layer "F.Cu") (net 30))
 (segment (start 107.785 155.360001) (end 107.66 155.235001) (width 0.2) (layer "F.Cu") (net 30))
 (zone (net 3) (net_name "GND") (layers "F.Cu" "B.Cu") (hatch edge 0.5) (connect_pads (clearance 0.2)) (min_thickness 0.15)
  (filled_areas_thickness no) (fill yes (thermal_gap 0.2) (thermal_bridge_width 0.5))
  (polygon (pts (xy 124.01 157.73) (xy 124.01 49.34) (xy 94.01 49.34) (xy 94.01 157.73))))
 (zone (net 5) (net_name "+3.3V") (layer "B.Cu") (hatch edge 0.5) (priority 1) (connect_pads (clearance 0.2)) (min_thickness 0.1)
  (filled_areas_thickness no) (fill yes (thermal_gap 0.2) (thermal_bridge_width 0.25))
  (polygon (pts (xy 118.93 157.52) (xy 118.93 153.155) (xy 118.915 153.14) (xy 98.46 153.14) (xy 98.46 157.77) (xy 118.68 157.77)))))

